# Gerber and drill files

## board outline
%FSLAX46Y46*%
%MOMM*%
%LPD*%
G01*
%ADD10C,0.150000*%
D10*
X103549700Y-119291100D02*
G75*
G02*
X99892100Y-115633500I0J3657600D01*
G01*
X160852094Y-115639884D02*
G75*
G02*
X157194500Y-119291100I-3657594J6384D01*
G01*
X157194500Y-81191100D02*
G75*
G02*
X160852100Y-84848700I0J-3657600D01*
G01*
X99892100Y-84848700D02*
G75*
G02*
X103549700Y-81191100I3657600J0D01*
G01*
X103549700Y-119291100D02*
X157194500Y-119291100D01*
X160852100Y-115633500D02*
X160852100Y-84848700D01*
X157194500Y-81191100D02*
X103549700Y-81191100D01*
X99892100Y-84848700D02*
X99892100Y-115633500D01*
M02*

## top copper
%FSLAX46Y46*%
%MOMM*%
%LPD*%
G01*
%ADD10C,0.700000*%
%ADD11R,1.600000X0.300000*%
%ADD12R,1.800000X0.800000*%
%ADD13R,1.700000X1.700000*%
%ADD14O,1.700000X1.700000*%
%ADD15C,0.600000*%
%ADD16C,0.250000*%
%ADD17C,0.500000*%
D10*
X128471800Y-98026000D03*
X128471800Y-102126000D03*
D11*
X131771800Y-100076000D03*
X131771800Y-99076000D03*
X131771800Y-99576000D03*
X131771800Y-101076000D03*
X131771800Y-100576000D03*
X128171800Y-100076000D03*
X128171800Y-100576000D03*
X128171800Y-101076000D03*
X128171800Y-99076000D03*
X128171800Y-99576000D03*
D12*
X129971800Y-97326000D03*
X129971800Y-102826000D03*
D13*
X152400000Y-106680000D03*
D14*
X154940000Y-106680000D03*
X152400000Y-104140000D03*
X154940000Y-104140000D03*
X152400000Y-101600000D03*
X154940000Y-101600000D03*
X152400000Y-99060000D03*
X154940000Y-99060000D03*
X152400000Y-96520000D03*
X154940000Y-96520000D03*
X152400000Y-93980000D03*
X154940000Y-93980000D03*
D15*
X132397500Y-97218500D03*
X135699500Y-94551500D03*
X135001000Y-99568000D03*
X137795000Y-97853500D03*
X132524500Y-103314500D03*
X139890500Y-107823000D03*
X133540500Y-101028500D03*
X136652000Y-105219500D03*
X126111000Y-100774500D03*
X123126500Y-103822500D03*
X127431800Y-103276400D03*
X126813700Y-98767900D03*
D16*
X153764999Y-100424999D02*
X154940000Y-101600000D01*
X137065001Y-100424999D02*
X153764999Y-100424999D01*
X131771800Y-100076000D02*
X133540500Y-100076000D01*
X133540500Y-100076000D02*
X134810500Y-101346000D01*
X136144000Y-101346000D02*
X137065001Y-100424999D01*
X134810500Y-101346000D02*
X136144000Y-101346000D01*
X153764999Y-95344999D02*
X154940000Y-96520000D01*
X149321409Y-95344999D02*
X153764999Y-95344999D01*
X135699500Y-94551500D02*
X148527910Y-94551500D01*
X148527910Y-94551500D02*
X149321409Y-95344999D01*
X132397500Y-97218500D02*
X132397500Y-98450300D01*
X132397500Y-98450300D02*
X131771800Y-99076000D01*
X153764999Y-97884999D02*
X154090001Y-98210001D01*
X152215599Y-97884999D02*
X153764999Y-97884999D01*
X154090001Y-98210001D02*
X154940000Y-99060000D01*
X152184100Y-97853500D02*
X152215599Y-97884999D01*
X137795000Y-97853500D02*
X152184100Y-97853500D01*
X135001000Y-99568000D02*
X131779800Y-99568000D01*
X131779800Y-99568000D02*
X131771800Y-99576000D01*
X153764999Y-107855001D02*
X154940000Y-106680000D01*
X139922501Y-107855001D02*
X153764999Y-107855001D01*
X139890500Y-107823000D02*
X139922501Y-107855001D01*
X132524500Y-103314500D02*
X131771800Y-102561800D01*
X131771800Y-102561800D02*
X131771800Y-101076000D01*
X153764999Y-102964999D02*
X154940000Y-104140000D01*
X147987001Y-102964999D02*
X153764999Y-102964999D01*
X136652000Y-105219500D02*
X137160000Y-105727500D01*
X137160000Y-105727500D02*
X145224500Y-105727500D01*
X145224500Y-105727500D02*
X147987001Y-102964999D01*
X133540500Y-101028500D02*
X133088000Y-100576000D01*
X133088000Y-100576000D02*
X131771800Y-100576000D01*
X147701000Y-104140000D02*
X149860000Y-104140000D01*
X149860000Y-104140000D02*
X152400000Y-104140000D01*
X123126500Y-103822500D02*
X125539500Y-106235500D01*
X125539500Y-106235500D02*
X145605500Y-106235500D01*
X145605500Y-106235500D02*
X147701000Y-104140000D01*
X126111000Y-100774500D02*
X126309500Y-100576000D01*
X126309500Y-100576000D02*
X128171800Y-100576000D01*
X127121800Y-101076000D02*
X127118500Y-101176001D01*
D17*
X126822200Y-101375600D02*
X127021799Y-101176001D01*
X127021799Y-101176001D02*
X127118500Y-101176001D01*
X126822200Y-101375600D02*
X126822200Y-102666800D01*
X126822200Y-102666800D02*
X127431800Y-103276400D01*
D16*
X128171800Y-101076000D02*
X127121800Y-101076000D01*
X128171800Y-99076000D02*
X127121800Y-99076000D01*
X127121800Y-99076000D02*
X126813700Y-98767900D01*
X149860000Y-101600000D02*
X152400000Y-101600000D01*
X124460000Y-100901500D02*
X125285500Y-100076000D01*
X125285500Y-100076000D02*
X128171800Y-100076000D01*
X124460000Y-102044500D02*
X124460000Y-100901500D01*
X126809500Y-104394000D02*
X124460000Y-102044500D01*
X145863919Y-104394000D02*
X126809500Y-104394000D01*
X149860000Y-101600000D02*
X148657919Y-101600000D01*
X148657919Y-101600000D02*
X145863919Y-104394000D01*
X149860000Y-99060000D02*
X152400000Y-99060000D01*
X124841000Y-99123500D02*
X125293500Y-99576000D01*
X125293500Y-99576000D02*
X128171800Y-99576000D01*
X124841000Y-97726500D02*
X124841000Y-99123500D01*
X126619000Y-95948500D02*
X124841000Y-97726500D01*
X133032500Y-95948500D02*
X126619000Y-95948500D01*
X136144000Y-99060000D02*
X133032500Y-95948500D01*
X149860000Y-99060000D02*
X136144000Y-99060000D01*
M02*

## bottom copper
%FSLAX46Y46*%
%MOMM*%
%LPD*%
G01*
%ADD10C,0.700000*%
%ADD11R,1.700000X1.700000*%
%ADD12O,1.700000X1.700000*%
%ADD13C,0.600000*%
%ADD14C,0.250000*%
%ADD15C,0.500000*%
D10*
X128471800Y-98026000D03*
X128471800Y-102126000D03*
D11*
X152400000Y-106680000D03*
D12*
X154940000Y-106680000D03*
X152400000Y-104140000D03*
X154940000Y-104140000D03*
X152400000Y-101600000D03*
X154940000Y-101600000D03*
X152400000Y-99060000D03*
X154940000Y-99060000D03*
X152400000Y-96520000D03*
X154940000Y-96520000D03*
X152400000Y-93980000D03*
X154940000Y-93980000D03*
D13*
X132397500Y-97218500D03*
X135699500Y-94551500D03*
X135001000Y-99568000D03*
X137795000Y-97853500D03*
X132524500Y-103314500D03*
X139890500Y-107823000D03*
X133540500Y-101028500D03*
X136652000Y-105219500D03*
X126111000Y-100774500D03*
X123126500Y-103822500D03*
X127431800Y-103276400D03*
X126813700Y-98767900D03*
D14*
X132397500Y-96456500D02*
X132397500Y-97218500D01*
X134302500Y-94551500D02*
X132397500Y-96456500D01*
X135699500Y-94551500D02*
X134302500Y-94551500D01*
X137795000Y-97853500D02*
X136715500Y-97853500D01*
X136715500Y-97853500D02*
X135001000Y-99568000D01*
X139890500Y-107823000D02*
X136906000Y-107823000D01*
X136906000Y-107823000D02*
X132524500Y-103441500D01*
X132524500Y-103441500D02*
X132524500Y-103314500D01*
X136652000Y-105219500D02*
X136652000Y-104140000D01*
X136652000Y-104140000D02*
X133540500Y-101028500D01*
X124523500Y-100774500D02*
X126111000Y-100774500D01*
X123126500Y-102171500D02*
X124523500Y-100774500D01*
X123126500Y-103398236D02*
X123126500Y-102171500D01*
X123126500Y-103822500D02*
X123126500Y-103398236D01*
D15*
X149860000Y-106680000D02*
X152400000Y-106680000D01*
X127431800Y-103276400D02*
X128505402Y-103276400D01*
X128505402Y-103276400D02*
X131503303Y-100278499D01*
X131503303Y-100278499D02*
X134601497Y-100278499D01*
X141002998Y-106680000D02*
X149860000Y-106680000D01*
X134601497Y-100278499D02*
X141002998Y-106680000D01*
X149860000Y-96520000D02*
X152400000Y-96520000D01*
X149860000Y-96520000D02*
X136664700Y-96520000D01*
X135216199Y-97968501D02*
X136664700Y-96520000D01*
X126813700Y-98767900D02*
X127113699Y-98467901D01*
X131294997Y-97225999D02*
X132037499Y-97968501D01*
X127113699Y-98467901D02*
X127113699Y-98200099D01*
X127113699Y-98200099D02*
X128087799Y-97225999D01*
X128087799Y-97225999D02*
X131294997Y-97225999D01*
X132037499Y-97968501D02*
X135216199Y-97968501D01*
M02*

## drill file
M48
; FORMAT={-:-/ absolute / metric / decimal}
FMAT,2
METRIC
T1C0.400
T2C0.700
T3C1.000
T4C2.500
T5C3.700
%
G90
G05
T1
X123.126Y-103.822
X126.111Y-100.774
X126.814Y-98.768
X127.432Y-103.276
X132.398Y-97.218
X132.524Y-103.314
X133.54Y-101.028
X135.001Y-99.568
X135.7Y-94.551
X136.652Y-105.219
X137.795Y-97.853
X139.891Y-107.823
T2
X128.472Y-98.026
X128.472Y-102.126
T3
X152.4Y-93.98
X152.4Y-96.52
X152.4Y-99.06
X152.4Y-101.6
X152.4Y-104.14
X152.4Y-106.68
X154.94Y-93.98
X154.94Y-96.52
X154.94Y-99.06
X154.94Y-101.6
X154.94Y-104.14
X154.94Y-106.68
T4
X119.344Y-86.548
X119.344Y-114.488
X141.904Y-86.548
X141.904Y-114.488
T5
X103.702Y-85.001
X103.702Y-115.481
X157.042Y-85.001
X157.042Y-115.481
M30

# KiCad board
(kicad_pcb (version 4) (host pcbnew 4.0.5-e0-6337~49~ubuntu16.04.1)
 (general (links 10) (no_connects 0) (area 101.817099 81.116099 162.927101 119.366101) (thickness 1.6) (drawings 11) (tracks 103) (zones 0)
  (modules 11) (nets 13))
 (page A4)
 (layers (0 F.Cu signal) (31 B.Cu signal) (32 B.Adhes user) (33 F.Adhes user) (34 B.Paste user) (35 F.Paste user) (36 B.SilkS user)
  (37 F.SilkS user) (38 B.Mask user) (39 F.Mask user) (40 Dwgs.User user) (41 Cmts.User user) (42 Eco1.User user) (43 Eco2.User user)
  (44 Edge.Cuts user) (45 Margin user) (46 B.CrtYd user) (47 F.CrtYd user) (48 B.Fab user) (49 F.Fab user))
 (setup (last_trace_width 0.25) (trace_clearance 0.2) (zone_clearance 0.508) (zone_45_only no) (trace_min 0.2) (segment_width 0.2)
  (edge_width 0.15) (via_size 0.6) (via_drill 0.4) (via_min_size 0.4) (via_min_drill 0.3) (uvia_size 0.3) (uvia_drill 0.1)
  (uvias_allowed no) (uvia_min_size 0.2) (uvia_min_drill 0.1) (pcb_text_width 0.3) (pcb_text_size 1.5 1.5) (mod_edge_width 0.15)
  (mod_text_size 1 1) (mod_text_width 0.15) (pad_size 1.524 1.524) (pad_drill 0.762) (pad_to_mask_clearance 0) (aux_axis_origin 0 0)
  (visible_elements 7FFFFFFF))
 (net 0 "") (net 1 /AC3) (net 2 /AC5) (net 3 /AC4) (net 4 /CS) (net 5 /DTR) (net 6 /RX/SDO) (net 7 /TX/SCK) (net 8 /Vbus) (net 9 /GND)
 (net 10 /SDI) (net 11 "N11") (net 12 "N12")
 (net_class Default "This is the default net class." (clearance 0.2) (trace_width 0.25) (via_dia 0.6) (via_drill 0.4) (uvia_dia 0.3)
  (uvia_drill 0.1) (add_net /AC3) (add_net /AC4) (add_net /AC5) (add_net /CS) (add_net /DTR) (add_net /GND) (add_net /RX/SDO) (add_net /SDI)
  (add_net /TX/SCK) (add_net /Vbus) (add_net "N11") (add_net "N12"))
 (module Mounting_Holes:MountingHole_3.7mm (layer F.Cu) (at 157.0421 85.0011)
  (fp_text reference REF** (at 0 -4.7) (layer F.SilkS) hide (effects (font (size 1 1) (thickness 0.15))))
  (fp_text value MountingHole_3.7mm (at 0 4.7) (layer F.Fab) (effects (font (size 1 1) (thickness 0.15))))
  (pad 1 np_thru_hole circle (at 0 0) (size 3.7 3.7) (drill 3.7) (layers *.Cu *.Mask)))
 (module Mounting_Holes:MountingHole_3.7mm (layer F.Cu) (at 157.0421 115.4811)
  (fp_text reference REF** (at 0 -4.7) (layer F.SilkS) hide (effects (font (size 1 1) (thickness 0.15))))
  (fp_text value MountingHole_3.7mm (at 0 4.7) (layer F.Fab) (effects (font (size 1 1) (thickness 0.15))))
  (pad 1 np_thru_hole circle (at 0 0) (size 3.7 3.7) (drill 3.7) (layers *.Cu *.Mask)))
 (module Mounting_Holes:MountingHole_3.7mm (layer F.Cu) (at 103.7021 115.4811)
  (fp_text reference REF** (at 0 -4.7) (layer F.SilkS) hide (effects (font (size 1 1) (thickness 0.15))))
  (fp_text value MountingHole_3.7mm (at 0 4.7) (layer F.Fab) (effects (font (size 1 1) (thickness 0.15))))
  (pad 1 np_thru_hole circle (at 0 0) (size 3.7 3.7) (drill 3.7) (layers *.Cu *.Mask)))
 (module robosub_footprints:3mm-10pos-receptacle (layer F.Cu) (at 129.9718 100.076 90)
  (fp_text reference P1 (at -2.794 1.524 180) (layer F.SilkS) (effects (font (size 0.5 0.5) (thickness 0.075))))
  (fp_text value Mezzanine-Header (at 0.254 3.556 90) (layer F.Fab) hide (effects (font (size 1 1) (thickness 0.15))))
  (pad "" thru_hole circle (at 2.05 -1.5 90) (size 0.7 0.7) (drill 0.7) (layers *.Cu *.Mask))
  (pad "" thru_hole circle (at -2.05 -1.5 90) (size 0.7 0.7) (drill 0.7) (layers *.Cu *.Mask))
  (pad 6 smd rect (at 0 1.8 90) (size 0.3 1.6) (layers F.Cu F.Paste F.Mask) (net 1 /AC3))
  (pad 10 smd rect (at 1 1.8 90) (size 0.3 1.6) (layers F.Cu F.Paste F.Mask) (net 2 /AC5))
  (pad 8 smd rect (at 0.5 1.8 90) (size 0.3 1.6) (layers F.Cu F.Paste F.Mask) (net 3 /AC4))
  (pad 2 smd rect (at -1 1.8 90) (size 0.3 1.6) (layers F.Cu F.Paste F.Mask) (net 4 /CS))
  (pad 4 smd rect (at -0.5 1.8 90) (size 0.3 1.6) (layers F.Cu F.Paste F.Mask) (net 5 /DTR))
  (pad 5 smd rect (at 0 -1.8 90) (size 0.3 1.6) (layers F.Cu F.Paste F.Mask) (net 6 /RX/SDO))
  (pad 3 smd rect (at -0.5 -1.8 90) (size 0.3 1.6) (layers F.Cu F.Paste F.Mask) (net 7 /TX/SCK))
  (pad 1 smd rect (at -1 -1.8 90) (size 0.3 1.6) (layers F.Cu F.Paste F.Mask) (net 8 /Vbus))
  (pad 9 smd rect (at 1 -1.8 90) (size 0.3 1.6) (layers F.Cu F.Paste F.Mask) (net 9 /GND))
  (pad 7 smd rect (at 0.5 -1.8 90) (size 0.3 1.6) (layers F.Cu F.Paste F.Mask) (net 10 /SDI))
  (pad "" smd rect (at 2.75 0 90) (size 0.8 1.8) (layers F.Cu F.Paste F.Mask))
  (pad "" smd rect (at -2.75 0 90) (size 0.8 1.8) (layers F.Cu F.Paste F.Mask)))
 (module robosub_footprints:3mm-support (layer F.Cu) (at 119.3442 86.548204)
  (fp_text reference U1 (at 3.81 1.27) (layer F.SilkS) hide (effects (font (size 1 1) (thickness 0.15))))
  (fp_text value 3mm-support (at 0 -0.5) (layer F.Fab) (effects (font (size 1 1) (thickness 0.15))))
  (pad "" np_thru_hole circle (at 0 0) (size 2.5 2.5) (drill 2.5) (layers *.Cu *.Mask)))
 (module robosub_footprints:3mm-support (layer F.Cu) (at 141.9042 86.548204)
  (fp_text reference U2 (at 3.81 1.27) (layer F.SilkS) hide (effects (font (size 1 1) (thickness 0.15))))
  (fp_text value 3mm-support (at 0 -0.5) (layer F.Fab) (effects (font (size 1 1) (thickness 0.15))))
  (pad "" np_thru_hole circle (at 0 0) (size 2.5 2.5) (drill 2.5) (layers *.Cu *.Mask)))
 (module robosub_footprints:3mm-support (layer F.Cu) (at 119.3442 114.488204)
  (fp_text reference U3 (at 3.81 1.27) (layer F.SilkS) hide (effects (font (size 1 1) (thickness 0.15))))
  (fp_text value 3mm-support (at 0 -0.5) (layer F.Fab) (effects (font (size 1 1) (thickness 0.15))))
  (pad "" np_thru_hole circle (at 0 0) (size 2.5 2.5) (drill 2.5) (layers *.Cu *.Mask)))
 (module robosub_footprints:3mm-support (layer F.Cu) (at 141.9042 114.488204)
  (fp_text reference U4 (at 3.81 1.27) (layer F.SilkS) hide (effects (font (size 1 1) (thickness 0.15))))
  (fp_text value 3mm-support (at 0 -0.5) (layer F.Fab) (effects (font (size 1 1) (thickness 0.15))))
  (pad "" np_thru_hole circle (at 0 0) (size 2.5 2.5) (drill 2.5) (layers *.Cu *.Mask)))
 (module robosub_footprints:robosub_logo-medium (layer F.Cu) (at 108.7374 89.9668 90)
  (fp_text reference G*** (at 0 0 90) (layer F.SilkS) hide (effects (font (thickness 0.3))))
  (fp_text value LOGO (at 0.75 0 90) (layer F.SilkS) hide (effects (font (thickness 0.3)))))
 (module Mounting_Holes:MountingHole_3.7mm (layer F.Cu) (at 103.7021 85.0011)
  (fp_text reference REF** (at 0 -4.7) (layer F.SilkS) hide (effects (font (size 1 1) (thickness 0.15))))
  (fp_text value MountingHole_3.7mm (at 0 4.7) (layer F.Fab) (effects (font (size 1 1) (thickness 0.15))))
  (pad 1 np_thru_hole circle (at 0 0) (size 3.7 3.7) (drill 3.7) (layers *.Cu *.Mask)))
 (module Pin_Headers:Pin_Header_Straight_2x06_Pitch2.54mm (layer B.Cu) (at 152.4 106.68)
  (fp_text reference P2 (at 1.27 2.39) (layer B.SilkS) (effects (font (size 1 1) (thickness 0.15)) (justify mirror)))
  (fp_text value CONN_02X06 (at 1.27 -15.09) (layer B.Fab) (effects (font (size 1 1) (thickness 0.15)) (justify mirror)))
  (pad 1 thru_hole rect (at 0 0) (size 1.7 1.7) (drill 1) (layers *.Cu *.Mask) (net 8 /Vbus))
  (pad 2 thru_hole oval (at 2.54 0) (size 1.7 1.7) (drill 1) (layers *.Cu *.Mask) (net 4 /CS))
  (pad 3 thru_hole oval (at 0 -2.54) (size 1.7 1.7) (drill 1) (layers *.Cu *.Mask) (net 7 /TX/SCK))
  (pad 4 thru_hole oval (at 2.54 -2.54) (size 1.7 1.7) (drill 1) (layers *.Cu *.Mask) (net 5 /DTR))
  (pad 5 thru_hole oval (at 0 -5.08) (size 1.7 1.7) (drill 1) (layers *.Cu *.Mask) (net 6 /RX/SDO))
  (pad 6 thru_hole oval (at 2.54 -5.08) (size 1.7 1.7) (drill 1) (layers *.Cu *.Mask) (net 1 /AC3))
  (pad 7 thru_hole oval (at 0 -7.62) (size 1.7 1.7) (drill 1) (layers *.Cu *.Mask) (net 10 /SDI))
  (pad 8 thru_hole oval (at 2.54 -7.62) (size 1.7 1.7) (drill 1) (layers *.Cu *.Mask) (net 3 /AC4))
  (pad 9 thru_hole oval (at 0 -10.16) (size 1.7 1.7) (drill 1) (layers *.Cu *.Mask) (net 9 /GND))
  (pad 10 thru_hole oval (at 2.54 -10.16) (size 1.7 1.7) (drill 1) (layers *.Cu *.Mask) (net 2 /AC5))
  (pad 11 thru_hole oval (at 0 -12.7) (size 1.7 1.7) (drill 1) (layers *.Cu *.Mask) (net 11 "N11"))
  (pad 12 thru_hole oval (at 2.54 -12.7) (size 1.7 1.7) (drill 1) (layers *.Cu *.Mask) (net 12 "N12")))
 (gr_arc (start 103.5497 115.6335) (end 99.8921 115.6335) (angle -90) (layer Edge.Cuts) (width 0.15))
 (gr_arc (start 157.1945 115.6335) (end 157.1945 119.2911) (angle -89.9) (layer Edge.Cuts) (width 0.15))
 (gr_arc (start 157.1945 84.8487) (end 160.8521 84.8487) (angle -90) (layer Edge.Cuts) (width 0.15))
 (gr_arc (start 103.5497 84.8487) (end 103.5497 81.1911) (angle -90) (layer Edge.Cuts) (width 0.15))
 (gr_line (start 103.5497 119.2911) (end 157.1945 119.2911) (layer Edge.Cuts) (width 0.15))
 (gr_line (start 160.8521 115.6335) (end 160.8521 84.8487) (layer Edge.Cuts) (width 0.15))
 (gr_line (start 157.1945 81.1911) (end 103.5497 81.1911) (layer Edge.Cuts) (width 0.15))
 (gr_line (start 99.8921 84.8487) (end 99.8921 115.6335) (layer Edge.Cuts) (width 0.15))
 (segment (start 153.764999 100.424999) (end 154.94 101.6) (width 0.25) (layer F.Cu) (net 1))
 (segment (start 137.065001 100.424999) (end 153.764999 100.424999) (width 0.25) (layer F.Cu) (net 1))
 (segment (start 131.7718 100.076) (end 133.5405 100.076) (width 0.25) (layer F.Cu) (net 1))
 (segment (start 133.5405 100.076) (end 134.8105 101.346) (width 0.25) (layer F.Cu) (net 1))
 (segment (start 136.144 101.346) (end 137.065001 100.424999) (width 0.25) (layer F.Cu) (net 1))
 (segment (start 134.8105 101.346) (end 136.144 101.346) (width 0.25) (layer F.Cu) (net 1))
 (segment (start 153.764999 95.344999) (end 154.94 96.52) (width 0.25) (layer F.Cu) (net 2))
 (segment (start 149.321409 95.344999) (end 153.764999 95.344999) (width 0.25) (layer F.Cu) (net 2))
 (segment (start 135.6995 94.5515) (end 148.52791 94.5515) (width 0.25) (layer F.Cu) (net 2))
 (segment (start 148.52791 94.5515) (end 149.321409 95.344999) (width 0.25) (layer F.Cu) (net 2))
 (segment (start 132.3975 97.2185) (end 132.3975 98.4503) (width 0.25) (layer F.Cu) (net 2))
 (segment (start 132.3975 98.4503) (end 131.7718 99.076) (width 0.25) (layer F.Cu) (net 2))
 (segment (start 132.3975 96.4565) (end 132.3975 97.2185) (width 0.25) (layer B.Cu) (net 2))
 (via (at 132.3975 97.2185) (size 0.6) (drill 0.4) (layers F.Cu B.Cu) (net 2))
 (segment (start 134.3025 94.5515) (end 132.3975 96.4565) (width 0.25) (layer B.Cu) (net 2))
 (segment (start 135.6995 94.5515) (end 134.3025 94.5515) (width 0.25) (layer B.Cu) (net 2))
 (via (at 135.6995 94.5515) (size 0.6) (drill 0.4) (layers F.Cu B.Cu) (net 2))
 (segment (start 153.764999 97.884999) (end 154.090001 98.210001) (width 0.25) (layer F.Cu) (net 3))
 (segment (start 152.215599 97.884999) (end 153.764999 97.884999) (width 0.25) (layer F.Cu) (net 3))
 (segment (start 154.090001 98.210001) (end 154.94 99.06) (width 0.25) (layer F.Cu) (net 3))
 (segment (start 152.1841 97.8535) (end 152.215599 97.884999) (width 0.25) (layer F.Cu) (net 3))
 (segment (start 137.795 97.8535) (end 152.1841 97.8535) (width 0.25) (layer F.Cu) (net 3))
 (segment (start 135.001 99.568) (end 131.7798 99.568) (width 0.25) (layer F.Cu) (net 3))
 (segment (start 131.7798 99.568) (end 131.7718 99.576) (width 0.25) (layer F.Cu) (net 3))
 (segment (start 137.795 97.8535) (end 136.7155 97.8535) (width 0.25) (layer B.Cu) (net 3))
 (segment (start 136.7155 97.8535) (end 135.001 99.568) (width 0.25) (layer B.Cu) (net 3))
 (via (at 135.001 99.568) (size 0.6) (drill 0.4) (layers F.Cu B.Cu) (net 3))
 (via (at 137.795 97.8535) (size 0.6) (drill 0.4) (layers F.Cu B.Cu) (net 3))
 (segment (start 153.764999 107.855001) (end 154.94 106.68) (width 0.25) (layer F.Cu) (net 4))
 (segment (start 139.922501 107.855001) (end 153.764999 107.855001) (width 0.25) (layer F.Cu) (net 4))
 (segment (start 139.8905 107.823) (end 139.922501 107.855001) (width 0.25) (layer F.Cu) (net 4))
 (segment (start 132.5245 103.3145) (end 131.7718 102.5618) (width 0.25) (layer F.Cu) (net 4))
 (segment (start 131.7718 102.5618) (end 131.7718 101.076) (width 0.25) (layer F.Cu) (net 4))
 (segment (start 139.8905 107.823) (end 136.906 107.823) (width 0.25) (layer B.Cu) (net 4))
 (segment (start 136.906 107.823) (end 132.5245 103.4415) (width 0.25) (layer B.Cu) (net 4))
 (segment (start 132.5245 103.4415) (end 132.5245 103.3145) (width 0.25) (layer B.Cu) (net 4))
 (via (at 132.5245 103.3145) (size 0.6) (drill 0.4) (layers F.Cu B.Cu) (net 4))
 (via (at 139.8905 107.823) (size 0.6) (drill 0.4) (layers F.Cu B.Cu) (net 4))
 (segment (start 153.764999 102.964999) (end 154.94 104.14) (width 0.25) (layer F.Cu) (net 5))
 (segment (start 147.987001 102.964999) (end 153.764999 102.964999) (width 0.25) (layer F.Cu) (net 5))
 (segment (start 136.652 105.2195) (end 137.16 105.7275) (width 0.25) (layer F.Cu) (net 5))
 (segment (start 137.16 105.7275) (end 145.2245 105.7275) (width 0.25) (layer F.Cu) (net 5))
 (segment (start 145.2245 105.7275) (end 147.987001 102.964999) (width 0.25) (layer F.Cu) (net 5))
 (segment (start 133.5405 101.0285) (end 133.088 100.576) (width 0.25) (layer F.Cu) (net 5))
 (segment (start 133.088 100.576) (end 131.7718 100.576) (width 0.25) (layer F.Cu) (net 5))
 (segment (start 136.652 105.2195) (end 136.652 104.14) (width 0.25) (layer B.Cu) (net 5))
 (segment (start 136.652 104.14) (end 133.5405 101.0285) (width 0.25) (layer B.Cu) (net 5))
 (via (at 133.5405 101.0285) (size 0.6) (drill 0.4) (layers F.Cu B.Cu) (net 5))
 (via (at 136.652 105.2195) (size 0.6) (drill 0.4) (layers F.Cu B.Cu) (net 5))
 (segment (start 147.701 104.14) (end 149.86 104.14) (width 0.25) (layer F.Cu) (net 7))
 (segment (start 149.86 104.14) (end 152.4 104.14) (width 0.25) (layer F.Cu) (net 7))
 (segment (start 123.1265 103.8225) (end 125.5395 106.2355) (width 0.25) (layer F.Cu) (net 7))
 (segment (start 125.5395 106.2355) (end 145.6055 106.2355) (width 0.25) (layer F.Cu) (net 7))
 (segment (start 145.6055 106.2355) (end 147.701 104.14) (width 0.25) (layer F.Cu) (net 7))
 (segment (start 126.111 100.7745) (end 126.3095 100.576) (width 0.25) (layer F.Cu) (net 7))
 (segment (start 126.3095 100.576) (end 128.1718 100.576) (width 0.25) (layer F.Cu) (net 7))
 (segment (start 124.5235 100.7745) (end 126.111 100.7745) (width 0.25) (layer B.Cu) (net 7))
 (via (at 126.111 100.7745) (size 0.6) (drill 0.4) (layers F.Cu B.Cu) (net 7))
 (segment (start 123.1265 102.1715) (end 124.5235 100.7745) (width 0.25) (layer B.Cu) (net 7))
 (segment (start 123.1265 103.398236) (end 123.1265 102.1715) (width 0.25) (layer B.Cu) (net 7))
 (segment (start 123.1265 103.8225) (end 123.1265 103.398236) (width 0.25) (layer B.Cu) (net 7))
 (via (at 123.1265 103.8225) (size 0.6) (drill 0.4) (layers F.Cu B.Cu) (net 7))
 (segment (start 149.86 106.68) (end 152.4 106.68) (width 0.5) (layer B.Cu) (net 8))
 (segment (start 127.4318 103.2764) (end 128.505402 103.2764) (width 0.5) (layer B.Cu) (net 8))
 (segment (start 128.505402 103.2764) (end 131.503303 100.278499) (width 0.5) (layer B.Cu) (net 8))
 (segment (start 131.503303 100.278499) (end 134.601497 100.278499) (width 0.5) (layer B.Cu) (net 8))
 (segment (start 141.002998 106.68) (end 149.86 106.68) (width 0.5) (layer B.Cu) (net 8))
 (segment (start 134.601497 100.278499) (end 141.002998 106.68) (width 0.5) (layer B.Cu) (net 8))
 (segment (start 127.1218 101.076) (end 127.1185 101.176001) (width 0.25) (layer F.Cu) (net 8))
 (segment (start 126.8222 101.3756) (end 127.021799 101.176001) (width 0.5) (layer F.Cu) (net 8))
 (segment (start 127.021799 101.176001) (end 127.1185 101.176001) (width 0.5) (layer F.Cu) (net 8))
 (segment (start 126.8222 101.3756) (end 126.8222 102.6668) (width 0.5) (layer F.Cu) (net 8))
 (segment (start 126.8222 102.6668) (end 127.4318 103.2764) (width 0.5) (layer F.Cu) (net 8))
 (via (at 127.4318 103.2764) (size 0.6) (drill 0.4) (layers F.Cu B.Cu) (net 8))
 (segment (start 128.1718 101.076) (end 127.1218 101.076) (width 0.25) (layer F.Cu) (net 8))
 (segment (start 149.86 96.52) (end 152.4 96.52) (width 0.5) (layer B.Cu) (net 9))
 (segment (start 149.86 96.52) (end 136.6647 96.52) (width 0.5) (layer B.Cu) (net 9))
 (segment (start 135.216199 97.968501) (end 136.6647 96.52) (width 0.5) (layer B.Cu) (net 9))
 (segment (start 126.8137 98.7679) (end 127.113699 98.467901) (width 0.5) (layer B.Cu) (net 9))
 (segment (start 131.294997 97.225999) (end 132.037499 97.968501) (width 0.5) (layer B.Cu) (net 9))
 (segment (start 127.113699 98.467901) (end 127.113699 98.200099) (width 0.5) (layer B.Cu) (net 9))
 (segment (start 127.113699 98.200099) (end 128.087799 97.225999) (width 0.5) (layer B.Cu) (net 9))
 (segment (start 128.087799 97.225999) (end 131.294997 97.225999) (width 0.5) (layer B.Cu) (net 9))
 (segment (start 132.037499 97.968501) (end 135.216199 97.968501) (width 0.5) (layer B.Cu) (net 9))
 (via (at 126.8137 98.7679) (size 0.6) (drill 0.4) (layers F.Cu B.Cu) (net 9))
 (segment (start 128.1718 99.076) (end 127.1218 99.076) (width 0.25) (layer F.Cu) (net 9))
 (segment (start 127.1218 99.076) (end 126.8137 98.7679) (width 0.25) (layer F.Cu) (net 9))
 (segment (start 149.86 101.6) (end 152.4 101.6) (width 0.25) (layer F.Cu) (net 6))
 (segment (start 124.46 100.9015) (end 125.2855 100.076) (width 0.25) (layer F.Cu) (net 6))
 (segment (start 125.2855 100.076) (end 128.1718 100.076) (width 0.25) (layer F.Cu) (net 6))
 (segment (start 124.46 102.0445) (end 124.46 100.9015) (width 0.25) (layer F.Cu) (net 6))
 (segment (start 126.8095 104.394) (end 124.46 102.0445) (width 0.25) (layer F.Cu) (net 6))
 (segment (start 145.863919 104.394) (end 126.8095 104.394) (width 0.25) (layer F.Cu) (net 6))
 (segment (start 149.86 101.6) (end 148.657919 101.6) (width 0.25) (layer F.Cu) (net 6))
 (segment (start 148.657919 101.6) (end 145.863919 104.394) (width 0.25) (layer F.Cu) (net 6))
 (segment (start 149.86 99.06) (end 152.4 99.06) (width 0.25) (layer F.Cu) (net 10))
 (segment (start 124.841 99.1235) (end 125.2935 99.576) (width 0.25) (layer F.Cu) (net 10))
 (segment (start 125.2935 99.576) (end 128.1718 99.576) (width 0.25) (layer F.Cu) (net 10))
 (segment (start 124.841 97.7265) (end 124.841 99.1235) (width 0.25) (layer F.Cu) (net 10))
 (segment (start 126.619 95.9485) (end 124.841 97.7265) (width 0.25) (layer F.Cu) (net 10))
 (segment (start 133.0325 95.9485) (end 126.619 95.9485) (width 0.25) (layer F.Cu) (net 10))
 (segment (start 136.144 99.06) (end 133.0325 95.9485) (width 0.25) (layer F.Cu) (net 10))
 (segment (start 149.86 99.06) (end 136.144 99.06) (width 0.25) (layer F.Cu) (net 10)))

